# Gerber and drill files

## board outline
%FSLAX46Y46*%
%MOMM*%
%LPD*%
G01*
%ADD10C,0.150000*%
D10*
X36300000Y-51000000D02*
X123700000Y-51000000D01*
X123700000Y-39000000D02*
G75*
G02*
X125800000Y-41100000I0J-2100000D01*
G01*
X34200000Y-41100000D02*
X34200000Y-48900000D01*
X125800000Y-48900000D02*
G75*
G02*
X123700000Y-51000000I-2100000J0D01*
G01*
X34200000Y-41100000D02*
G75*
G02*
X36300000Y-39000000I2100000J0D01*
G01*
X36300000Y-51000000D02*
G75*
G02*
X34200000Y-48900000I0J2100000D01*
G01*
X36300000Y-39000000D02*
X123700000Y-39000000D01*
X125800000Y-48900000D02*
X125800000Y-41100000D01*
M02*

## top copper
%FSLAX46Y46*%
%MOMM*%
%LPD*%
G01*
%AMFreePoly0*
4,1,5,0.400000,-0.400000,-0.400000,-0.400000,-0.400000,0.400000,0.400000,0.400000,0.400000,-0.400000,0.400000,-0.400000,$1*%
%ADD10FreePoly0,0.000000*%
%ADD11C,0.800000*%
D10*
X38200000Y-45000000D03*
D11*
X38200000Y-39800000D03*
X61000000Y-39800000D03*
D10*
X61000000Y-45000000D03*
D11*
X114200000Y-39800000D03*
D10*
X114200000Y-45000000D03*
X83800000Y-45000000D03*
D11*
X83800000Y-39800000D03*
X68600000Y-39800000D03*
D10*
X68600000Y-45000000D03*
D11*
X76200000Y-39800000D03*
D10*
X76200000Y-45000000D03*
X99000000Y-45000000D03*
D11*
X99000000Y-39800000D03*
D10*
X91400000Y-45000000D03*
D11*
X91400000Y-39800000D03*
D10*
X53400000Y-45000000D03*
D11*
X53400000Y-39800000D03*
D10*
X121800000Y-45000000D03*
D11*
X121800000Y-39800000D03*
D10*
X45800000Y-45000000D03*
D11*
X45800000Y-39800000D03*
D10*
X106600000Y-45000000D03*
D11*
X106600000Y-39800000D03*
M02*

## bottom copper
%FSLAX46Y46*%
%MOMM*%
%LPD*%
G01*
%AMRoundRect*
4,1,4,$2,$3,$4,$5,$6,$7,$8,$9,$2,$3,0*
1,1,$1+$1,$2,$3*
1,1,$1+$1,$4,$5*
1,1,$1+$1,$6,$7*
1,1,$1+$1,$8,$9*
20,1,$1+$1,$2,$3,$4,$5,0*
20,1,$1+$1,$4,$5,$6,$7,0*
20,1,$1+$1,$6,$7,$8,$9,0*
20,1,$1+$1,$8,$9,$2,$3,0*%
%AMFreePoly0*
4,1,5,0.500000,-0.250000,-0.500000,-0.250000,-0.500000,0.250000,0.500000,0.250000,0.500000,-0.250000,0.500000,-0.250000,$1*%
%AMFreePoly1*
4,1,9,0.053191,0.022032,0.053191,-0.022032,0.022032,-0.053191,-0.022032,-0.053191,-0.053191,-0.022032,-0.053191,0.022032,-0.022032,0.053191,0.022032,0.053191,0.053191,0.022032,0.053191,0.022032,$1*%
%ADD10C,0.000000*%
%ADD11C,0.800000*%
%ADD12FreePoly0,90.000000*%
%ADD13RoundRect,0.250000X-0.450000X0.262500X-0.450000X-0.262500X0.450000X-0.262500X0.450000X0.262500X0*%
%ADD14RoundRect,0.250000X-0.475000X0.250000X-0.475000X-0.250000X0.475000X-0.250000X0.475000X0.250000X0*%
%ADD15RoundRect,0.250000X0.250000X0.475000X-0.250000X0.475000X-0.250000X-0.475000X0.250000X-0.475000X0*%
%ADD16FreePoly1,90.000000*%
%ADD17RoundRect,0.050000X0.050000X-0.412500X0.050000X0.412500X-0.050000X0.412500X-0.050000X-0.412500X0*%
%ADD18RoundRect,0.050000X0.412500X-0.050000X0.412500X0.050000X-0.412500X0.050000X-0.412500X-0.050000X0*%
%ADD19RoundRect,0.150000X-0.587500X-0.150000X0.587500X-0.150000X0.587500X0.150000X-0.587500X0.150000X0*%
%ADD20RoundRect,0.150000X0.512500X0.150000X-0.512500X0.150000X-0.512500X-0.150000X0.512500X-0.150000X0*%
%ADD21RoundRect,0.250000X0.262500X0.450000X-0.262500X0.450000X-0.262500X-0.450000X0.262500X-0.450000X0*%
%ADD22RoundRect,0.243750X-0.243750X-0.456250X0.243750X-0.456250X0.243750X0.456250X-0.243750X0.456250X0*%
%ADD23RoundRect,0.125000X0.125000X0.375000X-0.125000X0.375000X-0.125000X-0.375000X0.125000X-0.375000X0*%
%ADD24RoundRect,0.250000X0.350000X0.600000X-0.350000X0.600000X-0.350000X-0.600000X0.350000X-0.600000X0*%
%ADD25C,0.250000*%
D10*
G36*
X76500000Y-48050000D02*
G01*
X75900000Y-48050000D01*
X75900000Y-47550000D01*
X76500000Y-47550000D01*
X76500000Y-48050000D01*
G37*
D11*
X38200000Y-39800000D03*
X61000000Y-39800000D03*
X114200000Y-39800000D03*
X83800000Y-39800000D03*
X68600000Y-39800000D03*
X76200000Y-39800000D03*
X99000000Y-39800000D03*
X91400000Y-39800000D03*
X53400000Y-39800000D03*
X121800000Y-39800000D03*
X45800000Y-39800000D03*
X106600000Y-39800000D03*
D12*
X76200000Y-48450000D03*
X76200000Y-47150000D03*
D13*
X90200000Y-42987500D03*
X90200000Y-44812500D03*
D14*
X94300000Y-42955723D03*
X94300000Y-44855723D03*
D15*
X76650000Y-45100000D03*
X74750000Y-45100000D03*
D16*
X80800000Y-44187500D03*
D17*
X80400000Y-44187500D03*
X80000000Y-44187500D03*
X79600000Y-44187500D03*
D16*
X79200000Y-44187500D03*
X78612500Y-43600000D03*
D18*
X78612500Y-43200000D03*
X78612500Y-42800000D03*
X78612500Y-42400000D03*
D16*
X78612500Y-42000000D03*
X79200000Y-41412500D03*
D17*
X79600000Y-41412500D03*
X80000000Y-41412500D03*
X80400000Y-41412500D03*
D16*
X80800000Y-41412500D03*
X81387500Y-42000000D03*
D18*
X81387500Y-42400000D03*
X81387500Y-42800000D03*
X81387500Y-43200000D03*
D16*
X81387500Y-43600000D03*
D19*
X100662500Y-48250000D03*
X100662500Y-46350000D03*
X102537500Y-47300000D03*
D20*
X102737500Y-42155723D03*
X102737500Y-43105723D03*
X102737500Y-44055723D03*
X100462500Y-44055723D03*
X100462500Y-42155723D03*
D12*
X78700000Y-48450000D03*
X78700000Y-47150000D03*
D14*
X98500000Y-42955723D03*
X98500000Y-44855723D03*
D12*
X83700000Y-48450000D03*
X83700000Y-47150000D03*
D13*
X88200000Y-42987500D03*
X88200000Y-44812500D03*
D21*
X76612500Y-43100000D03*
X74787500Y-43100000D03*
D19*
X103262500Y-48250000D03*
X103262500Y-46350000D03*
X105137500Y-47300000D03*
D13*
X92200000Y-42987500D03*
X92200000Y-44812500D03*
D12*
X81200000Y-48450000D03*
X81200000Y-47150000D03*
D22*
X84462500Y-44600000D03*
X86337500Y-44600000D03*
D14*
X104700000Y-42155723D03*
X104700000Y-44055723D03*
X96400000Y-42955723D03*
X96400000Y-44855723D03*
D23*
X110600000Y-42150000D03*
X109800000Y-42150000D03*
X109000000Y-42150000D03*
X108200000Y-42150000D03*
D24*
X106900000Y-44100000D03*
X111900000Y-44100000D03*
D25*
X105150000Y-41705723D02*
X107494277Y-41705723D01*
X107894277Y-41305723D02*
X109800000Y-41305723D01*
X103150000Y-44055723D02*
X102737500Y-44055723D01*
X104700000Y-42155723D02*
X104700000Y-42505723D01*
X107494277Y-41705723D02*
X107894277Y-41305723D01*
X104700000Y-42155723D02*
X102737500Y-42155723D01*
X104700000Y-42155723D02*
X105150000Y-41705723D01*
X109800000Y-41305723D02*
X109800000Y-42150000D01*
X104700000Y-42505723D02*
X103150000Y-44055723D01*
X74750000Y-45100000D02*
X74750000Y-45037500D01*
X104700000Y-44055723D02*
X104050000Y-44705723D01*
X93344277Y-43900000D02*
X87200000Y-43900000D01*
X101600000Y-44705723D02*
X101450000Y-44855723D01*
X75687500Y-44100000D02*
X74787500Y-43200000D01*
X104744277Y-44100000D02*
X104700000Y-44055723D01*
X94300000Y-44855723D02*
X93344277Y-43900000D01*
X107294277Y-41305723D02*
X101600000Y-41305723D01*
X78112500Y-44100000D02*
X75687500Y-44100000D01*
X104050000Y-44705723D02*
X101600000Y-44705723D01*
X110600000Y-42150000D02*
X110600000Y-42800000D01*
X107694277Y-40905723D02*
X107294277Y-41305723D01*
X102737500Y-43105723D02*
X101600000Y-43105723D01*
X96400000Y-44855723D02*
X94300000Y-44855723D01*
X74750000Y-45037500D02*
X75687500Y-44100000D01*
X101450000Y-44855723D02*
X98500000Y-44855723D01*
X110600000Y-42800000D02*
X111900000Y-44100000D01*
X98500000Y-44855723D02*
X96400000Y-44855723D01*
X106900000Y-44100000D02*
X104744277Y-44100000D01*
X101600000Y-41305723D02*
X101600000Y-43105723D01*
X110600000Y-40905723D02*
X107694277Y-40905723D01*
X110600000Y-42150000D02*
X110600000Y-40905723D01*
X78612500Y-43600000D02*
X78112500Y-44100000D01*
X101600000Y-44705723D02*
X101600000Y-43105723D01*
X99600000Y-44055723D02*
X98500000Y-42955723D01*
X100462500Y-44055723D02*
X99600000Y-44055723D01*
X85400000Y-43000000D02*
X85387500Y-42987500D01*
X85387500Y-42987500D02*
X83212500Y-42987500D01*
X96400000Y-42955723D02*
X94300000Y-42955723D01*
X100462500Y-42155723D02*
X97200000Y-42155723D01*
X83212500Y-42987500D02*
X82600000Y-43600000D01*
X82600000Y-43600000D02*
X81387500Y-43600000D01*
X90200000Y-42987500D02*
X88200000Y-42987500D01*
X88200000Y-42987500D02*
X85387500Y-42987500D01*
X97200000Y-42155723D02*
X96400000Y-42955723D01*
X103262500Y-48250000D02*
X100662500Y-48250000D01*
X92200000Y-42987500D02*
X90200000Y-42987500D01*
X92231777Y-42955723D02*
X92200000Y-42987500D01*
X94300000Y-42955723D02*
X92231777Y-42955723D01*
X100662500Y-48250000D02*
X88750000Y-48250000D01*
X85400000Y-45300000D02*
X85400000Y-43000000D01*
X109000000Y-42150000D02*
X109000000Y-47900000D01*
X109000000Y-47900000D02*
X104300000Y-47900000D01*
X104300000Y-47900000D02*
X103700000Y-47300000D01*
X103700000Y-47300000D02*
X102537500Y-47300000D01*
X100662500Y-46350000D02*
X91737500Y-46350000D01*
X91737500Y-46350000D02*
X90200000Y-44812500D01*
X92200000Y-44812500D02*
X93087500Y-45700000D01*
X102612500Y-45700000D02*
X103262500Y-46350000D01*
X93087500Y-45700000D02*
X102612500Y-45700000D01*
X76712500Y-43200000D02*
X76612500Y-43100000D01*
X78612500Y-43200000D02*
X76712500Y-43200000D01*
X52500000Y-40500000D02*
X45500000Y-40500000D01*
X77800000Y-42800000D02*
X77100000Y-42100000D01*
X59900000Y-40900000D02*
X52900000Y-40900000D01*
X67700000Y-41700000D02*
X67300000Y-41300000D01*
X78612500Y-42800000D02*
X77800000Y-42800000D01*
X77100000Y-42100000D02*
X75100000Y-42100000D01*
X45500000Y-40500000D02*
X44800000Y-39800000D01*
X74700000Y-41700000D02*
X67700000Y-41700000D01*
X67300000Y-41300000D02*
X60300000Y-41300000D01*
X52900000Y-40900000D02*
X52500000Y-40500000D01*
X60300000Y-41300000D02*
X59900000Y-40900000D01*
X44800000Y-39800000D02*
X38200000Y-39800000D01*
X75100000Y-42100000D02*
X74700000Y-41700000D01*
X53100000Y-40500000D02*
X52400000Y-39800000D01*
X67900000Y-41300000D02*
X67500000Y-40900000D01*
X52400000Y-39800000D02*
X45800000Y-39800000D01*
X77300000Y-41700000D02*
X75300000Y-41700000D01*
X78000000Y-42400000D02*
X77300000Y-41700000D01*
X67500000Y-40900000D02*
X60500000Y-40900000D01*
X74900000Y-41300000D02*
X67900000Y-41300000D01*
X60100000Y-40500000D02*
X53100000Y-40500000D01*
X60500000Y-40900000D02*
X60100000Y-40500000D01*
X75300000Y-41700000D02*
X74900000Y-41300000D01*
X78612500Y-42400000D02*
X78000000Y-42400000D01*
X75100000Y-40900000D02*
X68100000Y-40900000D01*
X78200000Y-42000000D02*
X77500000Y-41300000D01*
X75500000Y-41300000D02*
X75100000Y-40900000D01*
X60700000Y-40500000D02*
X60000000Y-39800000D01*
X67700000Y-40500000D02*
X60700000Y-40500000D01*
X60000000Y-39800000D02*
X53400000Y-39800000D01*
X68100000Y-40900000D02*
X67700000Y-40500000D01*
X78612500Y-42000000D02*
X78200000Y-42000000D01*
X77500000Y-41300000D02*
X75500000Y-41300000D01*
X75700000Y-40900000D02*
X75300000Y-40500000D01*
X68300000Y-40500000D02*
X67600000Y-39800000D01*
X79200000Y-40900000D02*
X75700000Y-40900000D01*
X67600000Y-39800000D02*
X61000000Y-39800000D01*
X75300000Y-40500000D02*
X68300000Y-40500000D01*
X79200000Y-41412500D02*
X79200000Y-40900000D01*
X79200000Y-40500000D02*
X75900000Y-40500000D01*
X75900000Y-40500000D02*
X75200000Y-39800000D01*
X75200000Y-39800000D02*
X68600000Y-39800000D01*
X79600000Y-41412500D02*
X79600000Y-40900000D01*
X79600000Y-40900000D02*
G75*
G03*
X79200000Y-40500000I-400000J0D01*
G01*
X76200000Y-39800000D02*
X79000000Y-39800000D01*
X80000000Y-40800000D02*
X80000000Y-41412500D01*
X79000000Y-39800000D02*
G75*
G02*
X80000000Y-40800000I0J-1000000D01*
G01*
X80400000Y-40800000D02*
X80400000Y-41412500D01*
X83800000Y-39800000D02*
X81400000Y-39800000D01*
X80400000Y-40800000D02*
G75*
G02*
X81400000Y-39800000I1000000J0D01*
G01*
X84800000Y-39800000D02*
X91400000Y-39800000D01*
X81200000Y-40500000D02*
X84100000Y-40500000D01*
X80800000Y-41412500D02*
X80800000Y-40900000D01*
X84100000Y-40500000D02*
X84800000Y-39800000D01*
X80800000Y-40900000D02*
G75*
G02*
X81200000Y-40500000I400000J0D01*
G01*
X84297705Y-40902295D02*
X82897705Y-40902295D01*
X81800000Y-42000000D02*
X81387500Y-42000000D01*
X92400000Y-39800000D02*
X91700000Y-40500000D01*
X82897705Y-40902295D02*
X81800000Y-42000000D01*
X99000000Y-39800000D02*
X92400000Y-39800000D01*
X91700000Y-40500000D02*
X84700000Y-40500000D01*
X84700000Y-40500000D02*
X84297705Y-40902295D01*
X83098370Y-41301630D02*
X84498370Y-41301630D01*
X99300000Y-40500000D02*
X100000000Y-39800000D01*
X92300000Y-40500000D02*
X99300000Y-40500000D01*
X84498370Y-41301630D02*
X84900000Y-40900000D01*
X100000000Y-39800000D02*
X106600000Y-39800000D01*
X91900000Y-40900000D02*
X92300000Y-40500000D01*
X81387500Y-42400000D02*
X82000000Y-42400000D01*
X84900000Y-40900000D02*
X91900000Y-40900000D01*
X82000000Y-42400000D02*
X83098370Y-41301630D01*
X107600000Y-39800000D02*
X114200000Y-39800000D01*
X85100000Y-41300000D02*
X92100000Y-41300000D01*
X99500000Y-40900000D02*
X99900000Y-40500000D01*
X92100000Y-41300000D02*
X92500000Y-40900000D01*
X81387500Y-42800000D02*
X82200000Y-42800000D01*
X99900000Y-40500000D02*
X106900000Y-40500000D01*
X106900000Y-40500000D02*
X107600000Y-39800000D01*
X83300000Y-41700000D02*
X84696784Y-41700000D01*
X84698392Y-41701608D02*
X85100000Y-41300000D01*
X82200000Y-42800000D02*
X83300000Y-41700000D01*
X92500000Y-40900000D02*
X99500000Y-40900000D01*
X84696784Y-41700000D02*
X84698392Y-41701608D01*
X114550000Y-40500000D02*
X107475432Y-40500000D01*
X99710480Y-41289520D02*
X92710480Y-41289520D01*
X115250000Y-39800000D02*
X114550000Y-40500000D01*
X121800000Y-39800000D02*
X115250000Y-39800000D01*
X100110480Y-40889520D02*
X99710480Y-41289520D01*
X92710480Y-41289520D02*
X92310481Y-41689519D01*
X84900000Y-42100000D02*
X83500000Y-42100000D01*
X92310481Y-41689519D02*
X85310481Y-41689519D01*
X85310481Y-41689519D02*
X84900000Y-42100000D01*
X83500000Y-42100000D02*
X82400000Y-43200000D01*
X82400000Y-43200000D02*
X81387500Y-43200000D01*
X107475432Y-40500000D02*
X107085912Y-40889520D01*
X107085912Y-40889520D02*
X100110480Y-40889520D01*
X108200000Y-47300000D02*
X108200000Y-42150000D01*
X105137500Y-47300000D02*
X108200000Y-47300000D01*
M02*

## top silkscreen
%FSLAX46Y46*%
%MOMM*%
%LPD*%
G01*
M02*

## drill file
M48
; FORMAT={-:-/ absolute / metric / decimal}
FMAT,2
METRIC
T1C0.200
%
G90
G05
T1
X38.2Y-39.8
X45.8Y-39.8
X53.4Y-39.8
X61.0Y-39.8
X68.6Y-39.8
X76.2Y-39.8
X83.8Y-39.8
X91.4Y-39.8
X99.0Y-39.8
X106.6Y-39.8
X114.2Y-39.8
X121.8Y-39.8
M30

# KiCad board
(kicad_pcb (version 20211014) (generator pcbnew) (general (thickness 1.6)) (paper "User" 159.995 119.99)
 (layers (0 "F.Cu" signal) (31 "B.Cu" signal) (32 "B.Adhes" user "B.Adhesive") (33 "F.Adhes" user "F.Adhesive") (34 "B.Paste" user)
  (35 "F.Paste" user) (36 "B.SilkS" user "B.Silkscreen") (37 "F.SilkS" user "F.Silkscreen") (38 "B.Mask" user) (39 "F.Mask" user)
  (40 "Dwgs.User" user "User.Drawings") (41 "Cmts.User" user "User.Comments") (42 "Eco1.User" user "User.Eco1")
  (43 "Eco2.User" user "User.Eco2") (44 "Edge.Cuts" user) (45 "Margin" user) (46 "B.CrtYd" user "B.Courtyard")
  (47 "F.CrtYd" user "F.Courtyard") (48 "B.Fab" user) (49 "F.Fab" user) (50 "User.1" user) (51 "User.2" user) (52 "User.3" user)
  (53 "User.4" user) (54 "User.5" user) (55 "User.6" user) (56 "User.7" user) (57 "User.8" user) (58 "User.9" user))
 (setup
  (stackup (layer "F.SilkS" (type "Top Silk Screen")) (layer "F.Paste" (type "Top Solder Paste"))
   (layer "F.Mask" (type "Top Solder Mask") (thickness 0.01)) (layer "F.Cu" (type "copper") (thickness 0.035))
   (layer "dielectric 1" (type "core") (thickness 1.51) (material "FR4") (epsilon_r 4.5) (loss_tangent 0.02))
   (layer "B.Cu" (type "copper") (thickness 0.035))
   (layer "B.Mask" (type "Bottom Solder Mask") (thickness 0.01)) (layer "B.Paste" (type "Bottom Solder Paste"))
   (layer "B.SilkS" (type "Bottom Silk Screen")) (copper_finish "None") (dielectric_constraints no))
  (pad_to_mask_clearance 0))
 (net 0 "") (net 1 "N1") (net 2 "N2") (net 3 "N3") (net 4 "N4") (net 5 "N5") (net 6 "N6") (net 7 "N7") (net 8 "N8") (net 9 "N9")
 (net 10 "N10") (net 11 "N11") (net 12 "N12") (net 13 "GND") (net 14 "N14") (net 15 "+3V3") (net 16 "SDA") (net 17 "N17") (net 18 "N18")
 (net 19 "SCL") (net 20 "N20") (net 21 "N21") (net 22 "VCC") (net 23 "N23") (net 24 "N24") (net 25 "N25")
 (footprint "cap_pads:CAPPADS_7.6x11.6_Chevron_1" (layer "F.Cu") (at 38.2 45)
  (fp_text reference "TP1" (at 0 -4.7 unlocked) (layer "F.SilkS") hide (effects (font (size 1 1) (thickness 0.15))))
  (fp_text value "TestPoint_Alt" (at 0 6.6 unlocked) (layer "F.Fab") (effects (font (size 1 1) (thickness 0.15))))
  (pad "1" smd custom (at 0 0) (size 0.8 0.8) (layers "F.Cu") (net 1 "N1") (options (clearance outline) (anchor rect)) (primitives))
  (pad "1" thru_hole circle (at 0 -5.2) (size 0.8 0.8) (drill 0.2) (layers *.Cu) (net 1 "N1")))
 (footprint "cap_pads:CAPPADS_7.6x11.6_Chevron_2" (layer "F.Cu") (at 61 45)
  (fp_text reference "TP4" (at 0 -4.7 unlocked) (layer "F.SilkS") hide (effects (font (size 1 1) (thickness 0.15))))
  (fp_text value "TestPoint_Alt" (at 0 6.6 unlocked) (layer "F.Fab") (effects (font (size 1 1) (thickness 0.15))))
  (pad "1" thru_hole circle (at 0 -5.2) (size 0.8 0.8) (drill 0.2) (layers *.Cu) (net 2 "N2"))
  (pad "1" smd custom (at 0 0) (size 0.8 0.8) (layers "F.Cu") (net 2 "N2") (options (clearance outline) (anchor rect)) (primitives)))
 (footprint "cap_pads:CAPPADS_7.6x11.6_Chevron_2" (layer "F.Cu") (at 114.2 45)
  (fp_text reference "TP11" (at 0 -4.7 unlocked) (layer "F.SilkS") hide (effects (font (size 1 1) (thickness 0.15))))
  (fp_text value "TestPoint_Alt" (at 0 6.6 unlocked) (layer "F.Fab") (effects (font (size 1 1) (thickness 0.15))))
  (pad "1" thru_hole circle (at 0 -5.2) (size 0.8 0.8) (drill 0.2) (layers *.Cu) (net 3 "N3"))
  (pad "1" smd custom (at 0 0) (size 0.8 0.8) (layers "F.Cu") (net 3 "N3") (options (clearance outline) (anchor rect)) (primitives)))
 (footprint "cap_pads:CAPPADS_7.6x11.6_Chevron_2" (layer "F.Cu") (at 83.8 45)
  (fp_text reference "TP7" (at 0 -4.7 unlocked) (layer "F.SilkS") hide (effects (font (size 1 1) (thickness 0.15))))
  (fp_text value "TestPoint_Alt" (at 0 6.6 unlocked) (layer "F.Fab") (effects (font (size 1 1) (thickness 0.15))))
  (pad "1" smd custom (at 0 0) (size 0.8 0.8) (layers "F.Cu") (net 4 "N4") (options (clearance outline) (anchor rect)) (primitives))
  (pad "1" thru_hole circle (at 0 -5.2) (size 0.8 0.8) (drill 0.2) (layers *.Cu) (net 4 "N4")))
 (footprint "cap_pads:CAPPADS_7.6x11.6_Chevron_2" (layer "F.Cu") (at 68.6 45)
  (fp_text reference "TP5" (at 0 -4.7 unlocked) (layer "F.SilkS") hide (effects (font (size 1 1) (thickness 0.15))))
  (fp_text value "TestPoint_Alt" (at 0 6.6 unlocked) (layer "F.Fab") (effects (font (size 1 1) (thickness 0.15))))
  (pad "1" thru_hole circle (at 0 -5.2) (size 0.8 0.8) (drill 0.2) (layers *.Cu) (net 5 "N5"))
  (pad "1" smd custom (at 0 0) (size 0.8 0.8) (layers "F.Cu") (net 5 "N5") (options (clearance outline) (anchor rect)) (primitives)))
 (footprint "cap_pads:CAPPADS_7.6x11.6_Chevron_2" (layer "F.Cu") (at 76.2 45)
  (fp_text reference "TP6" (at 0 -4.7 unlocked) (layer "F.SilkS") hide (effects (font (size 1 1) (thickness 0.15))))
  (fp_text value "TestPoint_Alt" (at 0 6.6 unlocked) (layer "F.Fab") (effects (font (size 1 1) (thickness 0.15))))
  (pad "1" thru_hole circle (at 0 -5.2) (size 0.8 0.8) (drill 0.2) (layers *.Cu) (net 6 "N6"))
  (pad "1" smd custom (at 0 0) (size 0.8 0.8) (layers "F.Cu") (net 6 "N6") (options (clearance outline) (anchor rect)) (primitives)))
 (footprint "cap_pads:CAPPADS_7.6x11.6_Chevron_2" (layer "F.Cu") (at 99 45)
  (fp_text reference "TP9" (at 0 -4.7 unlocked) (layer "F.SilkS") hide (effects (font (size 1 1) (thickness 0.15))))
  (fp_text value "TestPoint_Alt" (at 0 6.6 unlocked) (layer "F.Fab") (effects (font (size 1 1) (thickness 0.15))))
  (pad "1" smd custom (at 0 0) (size 0.8 0.8) (layers "F.Cu") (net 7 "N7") (options (clearance outline) (anchor rect)) (primitives))
  (pad "1" thru_hole circle (at 0 -5.2) (size 0.8 0.8) (drill 0.2) (layers *.Cu) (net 7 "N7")))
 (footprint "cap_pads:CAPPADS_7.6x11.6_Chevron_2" (layer "F.Cu") (at 91.4 45)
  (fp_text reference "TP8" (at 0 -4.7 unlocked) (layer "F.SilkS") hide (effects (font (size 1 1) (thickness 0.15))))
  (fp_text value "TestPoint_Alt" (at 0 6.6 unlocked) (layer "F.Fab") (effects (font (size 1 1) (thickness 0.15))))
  (pad "1" smd custom (at 0 0) (size 0.8 0.8) (layers "F.Cu") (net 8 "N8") (options (clearance outline) (anchor rect)) (primitives))
  (pad "1" thru_hole circle (at 0 -5.2) (size 0.8 0.8) (drill 0.2) (layers *.Cu) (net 8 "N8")))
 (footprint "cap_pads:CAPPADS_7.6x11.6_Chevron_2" (layer "F.Cu") (at 53.4 45)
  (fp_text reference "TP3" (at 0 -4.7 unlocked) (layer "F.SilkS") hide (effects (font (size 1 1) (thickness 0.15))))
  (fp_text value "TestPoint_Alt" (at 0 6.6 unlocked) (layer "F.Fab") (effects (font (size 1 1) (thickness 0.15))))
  (pad "1" smd custom (at 0 0) (size 0.8 0.8) (layers "F.Cu") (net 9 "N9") (options (clearance outline) (anchor rect)) (primitives))
  (pad "1" thru_hole circle (at 0 -5.2) (size 0.8 0.8) (drill 0.2) (layers *.Cu) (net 9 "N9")))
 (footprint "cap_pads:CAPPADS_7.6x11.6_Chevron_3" (layer "F.Cu") (at 121.8 45)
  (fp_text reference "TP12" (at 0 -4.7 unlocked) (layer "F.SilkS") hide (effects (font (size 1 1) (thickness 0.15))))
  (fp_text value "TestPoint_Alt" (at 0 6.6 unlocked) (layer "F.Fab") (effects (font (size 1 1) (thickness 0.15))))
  (pad "1" smd custom (at 0 0) (size 0.8 0.8) (layers "F.Cu") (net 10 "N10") (options (clearance outline) (anchor rect)) (primitives))
  (pad "1" thru_hole circle (at 0 -5.2) (size 0.8 0.8) (drill 0.2) (layers *.Cu) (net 10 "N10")))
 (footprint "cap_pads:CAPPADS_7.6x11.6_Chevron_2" (layer "F.Cu") (at 45.8 45)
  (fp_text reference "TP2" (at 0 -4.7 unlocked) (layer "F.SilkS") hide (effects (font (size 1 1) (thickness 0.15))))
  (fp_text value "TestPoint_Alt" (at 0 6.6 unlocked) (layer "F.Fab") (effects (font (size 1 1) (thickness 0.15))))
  (pad "1" smd custom (at 0 0) (size 0.8 0.8) (layers "F.Cu") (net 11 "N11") (options (clearance outline) (anchor rect)) (primitives))
  (pad "1" thru_hole circle (at 0 -5.2) (size 0.8 0.8) (drill 0.2) (layers *.Cu) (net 11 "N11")))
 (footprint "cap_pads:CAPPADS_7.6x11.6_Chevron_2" (layer "F.Cu") (at 106.6 45)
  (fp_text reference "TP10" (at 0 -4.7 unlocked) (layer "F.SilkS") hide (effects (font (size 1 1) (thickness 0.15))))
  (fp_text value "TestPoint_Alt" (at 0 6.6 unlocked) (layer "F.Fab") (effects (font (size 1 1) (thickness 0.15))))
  (pad "1" smd custom (at 0 0) (size 0.8 0.8) (layers "F.Cu") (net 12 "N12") (options (clearance outline) (anchor rect)) (primitives))
  (pad "1" thru_hole circle (at 0 -5.2) (size 0.8 0.8) (drill 0.2) (layers *.Cu) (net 12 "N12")))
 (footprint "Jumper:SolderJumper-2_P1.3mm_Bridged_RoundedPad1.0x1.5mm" (layer "B.Cu") (at 76.2 47.8 90)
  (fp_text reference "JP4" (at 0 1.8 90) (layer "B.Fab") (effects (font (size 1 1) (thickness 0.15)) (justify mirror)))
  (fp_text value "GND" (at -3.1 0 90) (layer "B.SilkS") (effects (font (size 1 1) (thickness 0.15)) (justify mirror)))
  (fp_poly (pts (xy 0.25 0.3) (xy -0.25 0.3) (xy -0.25 -0.3) (xy 0.25 -0.3)) (layer "B.Cu") (width 0) (fill solid))
  (pad "1" smd custom (at -0.65 0 90) (size 1 0.5) (layers "B.Cu" "B.Mask") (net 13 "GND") (zone_connect 2)
   (options (clearance outline) (anchor rect)) (primitives))
  (pad "2" smd custom (at 0.65 0 90) (size 1 0.5) (layers "B.Cu" "B.Mask") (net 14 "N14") (zone_connect 2)
   (options (clearance outline) (anchor rect)) (primitives)))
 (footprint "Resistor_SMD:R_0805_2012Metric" (layer "B.Cu") (at 90.2 43.9 -90)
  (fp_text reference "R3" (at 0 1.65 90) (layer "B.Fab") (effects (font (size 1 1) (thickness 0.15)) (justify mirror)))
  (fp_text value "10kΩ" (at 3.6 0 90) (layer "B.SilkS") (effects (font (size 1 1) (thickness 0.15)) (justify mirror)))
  (pad "1" smd roundrect (at -0.9125 0 270) (size 1.025 1.4) (layers "B.Cu" "B.Paste" "B.Mask") (roundrect_rratio 0.243902) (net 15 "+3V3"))
  (pad "2" smd roundrect (at 0.9125 0 270) (size 1.025 1.4) (layers "B.Cu" "B.Paste" "B.Mask") (roundrect_rratio 0.243902) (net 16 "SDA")))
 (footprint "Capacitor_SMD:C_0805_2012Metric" (layer "B.Cu") (at 94.3 43.905723 -90)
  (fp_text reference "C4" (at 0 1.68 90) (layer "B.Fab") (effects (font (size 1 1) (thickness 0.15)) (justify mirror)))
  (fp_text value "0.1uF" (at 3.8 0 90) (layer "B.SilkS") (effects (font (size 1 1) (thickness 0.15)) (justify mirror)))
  (pad "1" smd roundrect (at -0.95 0 270) (size 1 1.45) (layers "B.Cu" "B.Paste" "B.Mask") (roundrect_rratio 0.25) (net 15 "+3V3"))
  (pad "2" smd roundrect (at 0.95 0 270) (size 1 1.45) (layers "B.Cu" "B.Paste" "B.Mask") (roundrect_rratio 0.25) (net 13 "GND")))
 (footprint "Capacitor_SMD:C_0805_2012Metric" (layer "B.Cu") (at 75.7 45.1 180)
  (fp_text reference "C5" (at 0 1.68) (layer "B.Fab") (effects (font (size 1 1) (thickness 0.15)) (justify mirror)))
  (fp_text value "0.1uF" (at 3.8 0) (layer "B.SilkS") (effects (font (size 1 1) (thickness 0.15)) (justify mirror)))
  (pad "1" smd roundrect (at -0.95 0 180) (size 1 1.45) (layers "B.Cu" "B.Paste" "B.Mask") (roundrect_rratio 0.25) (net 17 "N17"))
  (pad "2" smd roundrect (at 0.95 0 180) (size 1 1.45) (layers "B.Cu" "B.Paste" "B.Mask") (roundrect_rratio 0.25) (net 13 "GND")))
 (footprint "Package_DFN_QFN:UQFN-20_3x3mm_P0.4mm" (layer "B.Cu") (at 80 42.8 90)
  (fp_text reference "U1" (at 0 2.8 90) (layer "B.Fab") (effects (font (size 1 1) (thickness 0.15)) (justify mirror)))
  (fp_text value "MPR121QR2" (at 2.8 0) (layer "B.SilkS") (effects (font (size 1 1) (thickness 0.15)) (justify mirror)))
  (pad "1" smd custom (at -1.3875 0.8 90) (size 0.115147 0.115147) (layers "B.Cu" "B.Paste" "B.Mask") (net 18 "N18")
   (options (clearance outline) (anchor circle)) (primitives))
  (pad "2" smd roundrect (at -1.3875 0.4 90) (size 0.925 0.2) (layers "B.Cu" "B.Paste" "B.Mask") (roundrect_rratio 0.25) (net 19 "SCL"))
  (pad "3" smd roundrect (at -1.3875 0 90) (size 0.925 0.2) (layers "B.Cu" "B.Paste" "B.Mask") (roundrect_rratio 0.25) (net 16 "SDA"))
  (pad "4" smd roundrect (at -1.3875 -0.4 90) (size 0.925 0.2) (layers "B.Cu" "B.Paste" "B.Mask") (roundrect_rratio 0.25) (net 14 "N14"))
  (pad "5" smd custom (at -1.3875 -0.8 90) (size 0.115147 0.115147) (layers "B.Cu" "B.Paste" "B.Mask") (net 17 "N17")
   (options (clearance outline) (anchor circle)) (primitives))
  (pad "6" smd custom (at -0.8 -1.3875 90) (size 0.115147 0.115147) (layers "B.Cu" "B.Paste" "B.Mask") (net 13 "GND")
   (options (clearance outline) (anchor circle)) (primitives))
  (pad "7" smd roundrect (at -0.4 -1.3875 90) (size 0.2 0.925) (layers "B.Cu" "B.Paste" "B.Mask") (roundrect_rratio 0.25) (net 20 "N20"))
  (pad "8" smd roundrect (at 0 -1.3875 90) (size 0.2 0.925) (layers "B.Cu" "B.Paste" "B.Mask") (roundrect_rratio 0.25) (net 1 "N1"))
  (pad "9" smd roundrect (at 0.4 -1.3875 90) (size 0.2 0.925) (layers "B.Cu" "B.Paste" "B.Mask") (roundrect_rratio 0.25) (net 11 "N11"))
  (pad "10" smd custom (at 0.8 -1.3875 90) (size 0.115147 0.115147) (layers "B.Cu" "B.Paste" "B.Mask") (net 9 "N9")
   (options (clearance outline) (anchor circle)) (primitives))
  (pad "11" smd custom (at 1.3875 -0.8 90) (size 0.115147 0.115147) (layers "B.Cu" "B.Paste" "B.Mask") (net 2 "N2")
   (options (clearance outline) (anchor circle)) (primitives))
  (pad "12" smd roundrect (at 1.3875 -0.4 90) (size 0.925 0.2) (layers "B.Cu" "B.Paste" "B.Mask") (roundrect_rratio 0.25) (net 5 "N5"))
  (pad "13" smd roundrect (at 1.3875 0 90) (size 0.925 0.2) (layers "B.Cu" "B.Paste" "B.Mask") (roundrect_rratio 0.25) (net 6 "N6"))
  (pad "14" smd roundrect (at 1.3875 0.4 90) (size 0.925 0.2) (layers "B.Cu" "B.Paste" "B.Mask") (roundrect_rratio 0.25) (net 4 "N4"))
  (pad "15" smd custom (at 1.3875 0.8 90) (size 0.115147 0.115147) (layers "B.Cu" "B.Paste" "B.Mask") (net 8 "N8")
   (options (clearance outline) (anchor circle)) (primitives))
  (pad "16" smd custom (at 0.8 1.3875 90) (size 0.115147 0.115147) (layers "B.Cu" "B.Paste" "B.Mask") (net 7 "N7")
   (options (clearance outline) (anchor circle)) (primitives))
  (pad "17" smd roundrect (at 0.4 1.3875 90) (size 0.2 0.925) (layers "B.Cu" "B.Paste" "B.Mask") (roundrect_rratio 0.25) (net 12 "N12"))
  (pad "18" smd roundrect (at 0 1.3875 90) (size 0.2 0.925) (layers "B.Cu" "B.Paste" "B.Mask") (roundrect_rratio 0.25) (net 3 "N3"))
  (pad "19" smd roundrect (at -0.4 1.3875 90) (size 0.2 0.925) (layers "B.Cu" "B.Paste" "B.Mask") (roundrect_rratio 0.25) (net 10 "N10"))
  (pad "20" smd custom (at -0.8 1.3875 90) (size 0.115147 0.115147) (layers "B.Cu" "B.Paste" "B.Mask") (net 15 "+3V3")
   (options (clearance outline) (anchor circle)) (primitives)))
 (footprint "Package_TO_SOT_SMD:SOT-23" (layer "B.Cu") (at 101.6 47.3)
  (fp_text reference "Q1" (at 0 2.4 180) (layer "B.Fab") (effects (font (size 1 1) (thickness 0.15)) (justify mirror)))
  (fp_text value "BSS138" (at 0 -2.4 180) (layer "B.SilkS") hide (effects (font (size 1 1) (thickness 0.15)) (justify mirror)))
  (pad "1" smd roundrect (at -0.9375 0.95) (size 1.475 0.6) (layers "B.Cu" "B.Paste" "B.Mask") (roundrect_rratio 0.25) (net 15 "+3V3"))
  (pad "2" smd roundrect (at -0.9375 -0.95) (size 1.475 0.6) (layers "B.Cu" "B.Paste" "B.Mask") (roundrect_rratio 0.25) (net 16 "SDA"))
  (pad "3" smd roundrect (at 0.9375 0) (size 1.475 0.6) (layers "B.Cu" "B.Paste" "B.Mask") (roundrect_rratio 0.25) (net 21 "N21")))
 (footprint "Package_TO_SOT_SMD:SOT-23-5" (layer "B.Cu") (at 101.6 43.105723 180)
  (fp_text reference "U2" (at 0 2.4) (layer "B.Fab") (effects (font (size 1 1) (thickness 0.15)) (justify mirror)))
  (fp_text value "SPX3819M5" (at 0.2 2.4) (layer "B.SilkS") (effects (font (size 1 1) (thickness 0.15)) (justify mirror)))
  (pad "1" smd roundrect (at -1.1375 0.95 180) (size 1.325 0.6) (layers "B.Cu" "B.Paste" "B.Mask") (roundrect_rratio 0.25) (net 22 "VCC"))
  (pad "2" smd roundrect (at -1.1375 0 180) (size 1.325 0.6) (layers "B.Cu" "B.Paste" "B.Mask") (roundrect_rratio 0.25) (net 13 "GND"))
  (pad "3" smd roundrect (at -1.1375 -0.95 180) (size 1.325 0.6) (layers "B.Cu" "B.Paste" "B.Mask") (roundrect_rratio 0.25) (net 22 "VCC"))
  (pad "4" smd roundrect (at 1.1375 -0.95 180) (size 1.325 0.6) (layers "B.Cu" "B.Paste" "B.Mask") (roundrect_rratio 0.25) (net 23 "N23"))
  (pad "5" smd roundrect (at 1.1375 0.95 180) (size 1.325 0.6) (layers "B.Cu" "B.Paste" "B.Mask") (roundrect_rratio 0.25) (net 15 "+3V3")))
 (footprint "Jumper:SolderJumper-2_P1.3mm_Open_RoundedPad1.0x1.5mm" (layer "B.Cu") (at 78.7 47.8 90)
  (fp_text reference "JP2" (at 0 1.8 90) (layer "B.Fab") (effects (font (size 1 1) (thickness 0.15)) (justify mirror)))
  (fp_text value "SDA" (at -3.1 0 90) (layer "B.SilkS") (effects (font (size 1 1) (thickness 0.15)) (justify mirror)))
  (pad "1" smd custom (at -0.65 0 90) (size 1 0.5) (layers "B.Cu" "B.Mask") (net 16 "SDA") (zone_connect 2)
   (options (clearance outline) (anchor rect)) (primitives))
  (pad "2" smd custom (at 0.65 0 90) (size 1 0.5) (layers "B.Cu" "B.Mask") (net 14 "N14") (zone_connect 2)
   (options (clearance outline) (anchor rect)) (primitives)))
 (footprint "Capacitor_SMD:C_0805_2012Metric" (layer "B.Cu") (at 98.5 43.905723 -90)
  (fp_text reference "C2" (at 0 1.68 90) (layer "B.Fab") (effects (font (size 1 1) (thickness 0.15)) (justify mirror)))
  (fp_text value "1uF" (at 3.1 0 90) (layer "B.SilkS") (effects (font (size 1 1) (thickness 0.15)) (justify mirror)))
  (pad "1" smd roundrect (at -0.95 0 270) (size 1 1.45) (layers "B.Cu" "B.Paste" "B.Mask") (roundrect_rratio 0.25) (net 23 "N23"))
  (pad "2" smd roundrect (at 0.95 0 270) (size 1 1.45) (layers "B.Cu" "B.Paste" "B.Mask") (roundrect_rratio 0.25) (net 13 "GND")))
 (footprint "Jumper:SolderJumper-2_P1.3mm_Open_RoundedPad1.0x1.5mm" (layer "B.Cu") (at 83.7 47.8 90)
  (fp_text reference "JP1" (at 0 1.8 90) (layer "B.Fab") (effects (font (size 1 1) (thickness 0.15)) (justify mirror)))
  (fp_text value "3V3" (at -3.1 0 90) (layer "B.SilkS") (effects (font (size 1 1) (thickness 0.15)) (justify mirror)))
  (pad "1" smd custom (at -0.65 0 90) (size 1 0.5) (layers "B.Cu" "B.Mask") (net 15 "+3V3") (zone_connect 2)
   (options (clearance outline) (anchor rect)) (primitives))
  (pad "2" smd custom (at 0.65 0 90) (size 1 0.5) (layers "B.Cu" "B.Mask") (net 14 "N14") (zone_connect 2)
   (options (clearance outline) (anchor rect)) (primitives)))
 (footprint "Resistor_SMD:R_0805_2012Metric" (layer "B.Cu") (at 88.2 43.9 -90)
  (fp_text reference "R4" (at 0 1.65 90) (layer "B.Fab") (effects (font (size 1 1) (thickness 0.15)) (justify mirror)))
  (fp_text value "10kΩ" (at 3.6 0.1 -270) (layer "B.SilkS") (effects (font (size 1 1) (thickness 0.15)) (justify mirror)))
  (pad "1" smd roundrect (at -0.9125 0 270) (size 1.025 1.4) (layers "B.Cu" "B.Paste" "B.Mask") (roundrect_rratio 0.243902) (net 15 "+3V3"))
  (pad "2" smd roundrect (at 0.9125 0 270) (size 1.025 1.4) (layers "B.Cu" "B.Paste" "B.Mask") (roundrect_rratio 0.243902) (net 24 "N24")))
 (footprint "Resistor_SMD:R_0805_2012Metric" (layer "B.Cu") (at 75.7 43.1 180)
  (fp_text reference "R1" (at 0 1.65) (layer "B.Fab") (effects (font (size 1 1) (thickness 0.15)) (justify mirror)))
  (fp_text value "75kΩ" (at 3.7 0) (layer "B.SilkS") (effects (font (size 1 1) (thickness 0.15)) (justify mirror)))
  (pad "1" smd roundrect (at -0.9125 0 180) (size 1.025 1.4) (layers "B.Cu" "B.Paste" "B.Mask") (roundrect_rratio 0.243902) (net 20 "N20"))
  (pad "2" smd roundrect (at 0.9125 0 180) (size 1.025 1.4) (layers "B.Cu" "B.Paste" "B.Mask") (roundrect_rratio 0.243902) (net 13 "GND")))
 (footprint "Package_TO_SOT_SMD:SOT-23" (layer "B.Cu") (at 104.2 47.3)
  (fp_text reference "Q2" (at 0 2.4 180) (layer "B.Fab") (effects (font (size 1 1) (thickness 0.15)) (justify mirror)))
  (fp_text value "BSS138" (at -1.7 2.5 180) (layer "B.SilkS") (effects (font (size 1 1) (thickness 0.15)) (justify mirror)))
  (pad "1" smd roundrect (at -0.9375 0.95) (size 1.475 0.6) (layers "B.Cu" "B.Paste" "B.Mask") (roundrect_rratio 0.25) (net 15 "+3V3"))
  (pad "2" smd roundrect (at -0.9375 -0.95) (size 1.475 0.6) (layers "B.Cu" "B.Paste" "B.Mask") (roundrect_rratio 0.25) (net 19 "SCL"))
  (pad "3" smd roundrect (at 0.9375 0) (size 1.475 0.6) (layers "B.Cu" "B.Paste" "B.Mask") (roundrect_rratio 0.25) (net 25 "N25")))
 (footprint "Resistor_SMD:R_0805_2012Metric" (layer "B.Cu") (at 92.2 43.9 -90)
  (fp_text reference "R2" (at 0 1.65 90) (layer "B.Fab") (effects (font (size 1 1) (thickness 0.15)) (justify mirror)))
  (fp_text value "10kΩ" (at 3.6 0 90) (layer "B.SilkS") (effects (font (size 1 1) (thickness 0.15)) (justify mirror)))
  (pad "1" smd roundrect (at -0.9125 0 270) (size 1.025 1.4) (layers "B.Cu" "B.Paste" "B.Mask") (roundrect_rratio 0.243902) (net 15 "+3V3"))
  (pad "2" smd roundrect (at 0.9125 0 270) (size 1.025 1.4) (layers "B.Cu" "B.Paste" "B.Mask") (roundrect_rratio 0.243902) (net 19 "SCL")))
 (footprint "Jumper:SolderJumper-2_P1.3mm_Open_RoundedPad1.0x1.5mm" (layer "B.Cu") (at 81.2 47.8 90)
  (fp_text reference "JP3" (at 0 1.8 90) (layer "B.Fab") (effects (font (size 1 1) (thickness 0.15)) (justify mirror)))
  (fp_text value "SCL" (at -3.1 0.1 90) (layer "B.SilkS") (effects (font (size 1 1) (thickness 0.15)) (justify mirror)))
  (pad "1" smd custom (at -0.65 0 90) (size 1 0.5) (layers "B.Cu" "B.Mask") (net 19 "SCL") (zone_connect 2)
   (options (clearance outline) (anchor rect)) (primitives))
  (pad "2" smd custom (at 0.65 0 90) (size 1 0.5) (layers "B.Cu" "B.Mask") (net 14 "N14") (zone_connect 2)
   (options (clearance outline) (anchor rect)) (primitives)))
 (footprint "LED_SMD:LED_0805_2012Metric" (layer "B.Cu") (at 85.4 44.6)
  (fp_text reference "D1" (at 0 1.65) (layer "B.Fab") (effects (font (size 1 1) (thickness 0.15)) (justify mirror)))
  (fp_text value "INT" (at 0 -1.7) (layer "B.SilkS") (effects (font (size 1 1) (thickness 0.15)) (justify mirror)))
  (pad "1" smd roundrect (at -0.9375 0) (size 0.975 1.4) (layers "B.Cu" "B.Paste" "B.Mask") (roundrect_rratio 0.25) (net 18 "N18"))
  (pad "2" smd roundrect (at 0.9375 0) (size 0.975 1.4) (layers "B.Cu" "B.Paste" "B.Mask") (roundrect_rratio 0.25) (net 24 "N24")))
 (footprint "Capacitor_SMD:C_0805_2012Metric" (layer "B.Cu") (at 104.7 43.105723 -90)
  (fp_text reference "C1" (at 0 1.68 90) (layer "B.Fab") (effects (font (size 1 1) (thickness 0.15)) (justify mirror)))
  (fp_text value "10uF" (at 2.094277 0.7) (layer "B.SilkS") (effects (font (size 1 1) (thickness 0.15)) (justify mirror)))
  (pad "1" smd roundrect (at -0.95 0 270) (size 1 1.45) (layers "B.Cu" "B.Paste" "B.Mask") (roundrect_rratio 0.25) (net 22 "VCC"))
  (pad "2" smd roundrect (at 0.95 0 270) (size 1 1.45) (layers "B.Cu" "B.Paste" "B.Mask") (roundrect_rratio 0.25) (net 13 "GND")))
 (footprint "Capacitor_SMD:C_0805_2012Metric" (layer "B.Cu") (at 96.4 43.905723 -90)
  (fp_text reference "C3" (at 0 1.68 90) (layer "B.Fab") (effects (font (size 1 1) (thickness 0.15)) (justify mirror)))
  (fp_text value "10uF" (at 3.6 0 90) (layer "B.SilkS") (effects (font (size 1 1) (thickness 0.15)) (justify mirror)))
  (pad "1" smd roundrect (at -0.95 0 270) (size 1 1.45) (layers "B.Cu" "B.Paste" "B.Mask") (roundrect_rratio 0.25) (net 15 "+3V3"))
  (pad "2" smd roundrect (at 0.95 0 270) (size 1 1.45) (layers "B.Cu" "B.Paste" "B.Mask") (roundrect_rratio 0.25) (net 13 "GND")))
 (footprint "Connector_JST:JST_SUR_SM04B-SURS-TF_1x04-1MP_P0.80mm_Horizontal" (layer "B.Cu") (at 109.4 43.3 180)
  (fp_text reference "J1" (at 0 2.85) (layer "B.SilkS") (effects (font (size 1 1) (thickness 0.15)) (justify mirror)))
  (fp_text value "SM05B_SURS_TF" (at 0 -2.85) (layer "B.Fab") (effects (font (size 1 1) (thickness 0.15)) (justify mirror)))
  (pad "1" smd roundrect (at -1.2 1.15 180) (size 0.5 1) (layers "B.Cu" "B.Paste" "B.Mask") (roundrect_rratio 0.25) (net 13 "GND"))
  (pad "2" smd roundrect (at -0.4 1.15 180) (size 0.5 1) (layers "B.Cu" "B.Paste" "B.Mask") (roundrect_rratio 0.25) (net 22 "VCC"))
  (pad "3" smd roundrect (at 0.4 1.15 180) (size 0.5 1) (layers "B.Cu" "B.Paste" "B.Mask") (roundrect_rratio 0.25) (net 21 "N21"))
  (pad "4" smd roundrect (at 1.2 1.15 180) (size 0.5 1) (layers "B.Cu" "B.Paste" "B.Mask") (roundrect_rratio 0.25) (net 25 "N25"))
  (pad "MP" smd roundrect (at 2.5 -0.8 180) (size 1.2 1.7) (layers "B.Cu" "B.Paste" "B.Mask") (roundrect_rratio 0.208333) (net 13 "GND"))
  (pad "MP" smd roundrect (at -2.5 -0.8 180) (size 1.2 1.7) (layers "B.Cu" "B.Paste" "B.Mask") (roundrect_rratio 0.208333) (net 13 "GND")))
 (gr_line (start 36.3 51) (end 123.7 51) (layer "Edge.Cuts") (width 0.15))
 (gr_arc (start 123.7 39) (mid 125.184924 39.615076) (end 125.8 41.1) (layer "Edge.Cuts") (width 0.15))
 (gr_line (start 34.2 41.1) (end 34.2 48.9) (layer "Edge.Cuts") (width 0.15))
 (gr_arc (start 125.8 48.9) (mid 125.184924 50.384924) (end 123.7 51) (layer "Edge.Cuts") (width 0.15))
 (gr_arc (start 34.2 41.1) (mid 34.815076 39.615076) (end 36.3 39) (layer "Edge.Cuts") (width 0.15))
 (gr_arc (start 36.3 51) (mid 34.815076 50.384924) (end 34.2 48.9) (layer "Edge.Cuts") (width 0.15))
 (gr_line (start 36.3 39) (end 123.7 39) (layer "Edge.Cuts") (width 0.15))
 (gr_line (start 125.8 48.9) (end 125.8 41.1) (layer "Edge.Cuts") (width 0.15))
 (segment (start 105.15 41.705723) (end 107.494277 41.705723) (width 0.25) (layer "B.Cu") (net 22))
 (segment (start 107.894277 41.305723) (end 109.8 41.305723) (width 0.25) (layer "B.Cu") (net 22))
 (segment (start 103.15 44.055723) (end 102.7375 44.055723) (width 0.25) (layer "B.Cu") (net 22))
 (segment (start 104.7 42.155723) (end 104.7 42.505723) (width 0.25) (layer "B.Cu") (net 22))
 (segment (start 107.494277 41.705723) (end 107.894277 41.305723) (width 0.25) (layer "B.Cu") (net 22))
 (segment (start 104.7 42.155723) (end 102.7375 42.155723) (width 0.25) (layer "B.Cu") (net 22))
 (segment (start 104.7 42.155723) (end 105.15 41.705723) (width 0.25) (layer "B.Cu") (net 22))
 (segment (start 109.8 41.305723) (end 109.8 42.15) (width 0.25) (layer "B.Cu") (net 22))
 (segment (start 104.7 42.505723) (end 103.15 44.055723) (width 0.25) (layer "B.Cu") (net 22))
 (segment (start 74.75 45.1) (end 74.75 45.0375) (width 0.25) (layer "B.Cu") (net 13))
 (segment (start 104.7 44.055723) (end 104.05 44.705723) (width 0.25) (layer "B.Cu") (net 13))
 (segment (start 93.344277 43.9) (end 87.2 43.9) (width 0.25) (layer "B.Cu") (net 13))
 (segment (start 101.6 44.705723) (end 101.45 44.855723) (width 0.25) (layer "B.Cu") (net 13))
 (segment (start 75.6875 44.1) (end 74.7875 43.2) (width 0.25) (layer "B.Cu") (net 13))
 (segment (start 104.744277 44.1) (end 104.7 44.055723) (width 0.25) (layer "B.Cu") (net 13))
 (segment (start 94.3 44.855723) (end 93.344277 43.9) (width 0.25) (layer "B.Cu") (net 13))
 (segment (start 107.294277 41.305723) (end 101.6 41.305723) (width 0.25) (layer "B.Cu") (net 13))
 (segment (start 78.1125 44.1) (end 75.6875 44.1) (width 0.25) (layer "B.Cu") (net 13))
 (segment (start 104.05 44.705723) (end 101.6 44.705723) (width 0.25) (layer "B.Cu") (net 13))
 (segment (start 110.6 42.15) (end 110.6 42.8) (width 0.25) (layer "B.Cu") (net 13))
 (segment (start 107.694277 40.905723) (end 107.294277 41.305723) (width 0.25) (layer "B.Cu") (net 13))
 (segment (start 102.7375 43.105723) (end 101.6 43.105723) (width 0.25) (layer "B.Cu") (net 13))
 (segment (start 96.4 44.855723) (end 94.3 44.855723) (width 0.25) (layer "B.Cu") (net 13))
 (segment (start 74.75 45.0375) (end 75.6875 44.1) (width 0.25) (layer "B.Cu") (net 13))
 (segment (start 101.45 44.855723) (end 98.5 44.855723) (width 0.25) (layer "B.Cu") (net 13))
 (segment (start 110.6 42.8) (end 111.9 44.1) (width 0.25) (layer "B.Cu") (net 13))
 (segment (start 98.5 44.855723) (end 96.4 44.855723) (width 0.25) (layer "B.Cu") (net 13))
 (segment (start 106.9 44.1) (end 104.744277 44.1) (width 0.25) (layer "B.Cu") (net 13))
 (segment (start 101.6 41.305723) (end 101.6 43.105723) (width 0.25) (layer "B.Cu") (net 13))
 (segment (start 110.6 40.905723) (end 107.694277 40.905723) (width 0.25) (layer "B.Cu") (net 13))
 (segment (start 110.6 42.15) (end 110.6 40.905723) (width 0.25) (layer "B.Cu") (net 13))
 (segment (start 78.6125 43.6) (end 78.1125 44.1) (width 0.25) (layer "B.Cu") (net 13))
 (segment (start 101.6 44.705723) (end 101.6 43.105723) (width 0.25) (layer "B.Cu") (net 13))
 (segment (start 99.6 44.055723) (end 98.5 42.955723) (width 0.25) (layer "B.Cu") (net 23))
 (segment (start 100.4625 44.055723) (end 99.6 44.055723) (width 0.25) (layer "B.Cu") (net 23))
 (segment (start 85.4 43) (end 85.3875 42.9875) (width 0.25) (layer "B.Cu") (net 15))
 (segment (start 85.3875 42.9875) (end 83.2125 42.9875) (width 0.25) (layer "B.Cu") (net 15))
 (segment (start 96.4 42.955723) (end 94.3 42.955723) (width 0.25) (layer "B.Cu") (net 15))
 (segment (start 100.4625 42.155723) (end 97.2 42.155723) (width 0.25) (layer "B.Cu") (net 15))
 (segment (start 83.2125 42.9875) (end 82.6 43.6) (width 0.25) (layer "B.Cu") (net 15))
 (segment (start 82.6 43.6) (end 81.3875 43.6) (width 0.25) (layer "B.Cu") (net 15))
 (segment (start 90.2 42.9875) (end 88.2 42.9875) (width 0.25) (layer "B.Cu") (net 15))
 (segment (start 88.2 42.9875) (end 85.3875 42.9875) (width 0.25) (layer "B.Cu") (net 15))
 (segment (start 97.2 42.155723) (end 96.4 42.955723) (width 0.25) (layer "B.Cu") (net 15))
 (segment (start 103.2625 48.25) (end 100.6625 48.25) (width 0.25) (layer "B.Cu") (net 15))
 (segment (start 92.2 42.9875) (end 90.2 42.9875) (width 0.25) (layer "B.Cu") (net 15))
 (segment (start 92.231777 42.955723) (end 92.2 42.9875) (width 0.25) (layer "B.Cu") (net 15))
 (segment (start 94.3 42.955723) (end 92.231777 42.955723) (width 0.25) (layer "B.Cu") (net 15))
 (segment (start 100.6625 48.25) (end 88.75 48.25) (width 0.25) (layer "B.Cu") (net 15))
 (segment (start 85.4 45.3) (end 85.4 43) (width 0.25) (layer "B.Cu") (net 15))
 (segment (start 109 42.15) (end 109 47.9) (width 0.25) (layer "B.Cu") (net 21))
 (segment (start 109 47.9) (end 104.3 47.9) (width 0.25) (layer "B.Cu") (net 21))
 (segment (start 104.3 47.9) (end 103.7 47.3) (width 0.25) (layer "B.Cu") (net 21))
 (segment (start 103.7 47.3) (end 102.5375 47.3) (width 0.25) (layer "B.Cu") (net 21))
 (segment (start 100.6625 46.35) (end 91.7375 46.35) (width 0.25) (layer "B.Cu") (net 16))
 (segment (start 91.7375 46.35) (end 90.2 44.8125) (width 0.25) (layer "B.Cu") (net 16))
 (segment (start 92.2 44.8125) (end 93.0875 45.7) (width 0.25) (layer "B.Cu") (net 19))
 (segment (start 102.6125 45.7) (end 103.2625 46.35) (width 0.25) (layer "B.Cu") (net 19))
 (segment (start 93.0875 45.7) (end 102.6125 45.7) (width 0.25) (layer "B.Cu") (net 19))
 (segment (start 76.7125 43.2) (end 76.6125 43.1) (width 0.25) (layer "B.Cu") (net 20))
 (segment (start 78.6125 43.2) (end 76.7125 43.2) (width 0.25) (layer "B.Cu") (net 20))
 (segment (start 52.5 40.5) (end 45.5 40.5) (width 0.25) (layer "B.Cu") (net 1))
 (segment (start 77.8 42.8) (end 77.1 42.1) (width 0.25) (layer "B.Cu") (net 1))
 (segment (start 59.9 40.9) (end 52.9 40.9) (width 0.25) (layer "B.Cu") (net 1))
 (segment (start 67.7 41.7) (end 67.3 41.3) (width 0.25) (layer "B.Cu") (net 1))
 (segment (start 78.6125 42.8) (end 77.8 42.8) (width 0.25) (layer "B.Cu") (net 1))
 (segment (start 77.1 42.1) (end 75.1 42.1) (width 0.25) (layer "B.Cu") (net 1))
 (segment (start 45.5 40.5) (end 44.8 39.8) (width 0.25) (layer "B.Cu") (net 1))
 (segment (start 74.7 41.7) (end 67.7 41.7) (width 0.25) (layer "B.Cu") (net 1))
 (segment (start 67.3 41.3) (end 60.3 41.3) (width 0.25) (layer "B.Cu") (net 1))
 (segment (start 52.9 40.9) (end 52.5 40.5) (width 0.25) (layer "B.Cu") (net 1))
 (segment (start 60.3 41.3) (end 59.9 40.9) (width 0.25) (layer "B.Cu") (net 1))
 (segment (start 44.8 39.8) (end 38.2 39.8) (width 0.25) (layer "B.Cu") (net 1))
 (segment (start 75.1 42.1) (end 74.7 41.7) (width 0.25) (layer "B.Cu") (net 1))
 (segment (start 53.1 40.5) (end 52.4 39.8) (width 0.25) (layer "B.Cu") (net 11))
 (segment (start 67.9 41.3) (end 67.5 40.9) (width 0.25) (layer "B.Cu") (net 11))
 (segment (start 52.4 39.8) (end 45.8 39.8) (width 0.25) (layer "B.Cu") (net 11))
 (segment (start 77.3 41.7) (end 75.3 41.7) (width 0.25) (layer "B.Cu") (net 11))
 (segment (start 78 42.4) (end 77.3 41.7) (width 0.25) (layer "B.Cu") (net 11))
 (segment (start 67.5 40.9) (end 60.5 40.9) (width 0.25) (layer "B.Cu") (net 11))
 (segment (start 74.9 41.3) (end 67.9 41.3) (width 0.25) (layer "B.Cu") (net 11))
 (segment (start 60.1 40.5) (end 53.1 40.5) (width 0.25) (layer "B.Cu") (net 11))
 (segment (start 60.5 40.9) (end 60.1 40.5) (width 0.25) (layer "B.Cu") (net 11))
 (segment (start 75.3 41.7) (end 74.9 41.3) (width 0.25) (layer "B.Cu") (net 11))
 (segment (start 78.6125 42.4) (end 78 42.4) (width 0.25) (layer "B.Cu") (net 11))
 (segment (start 75.1 40.9) (end 68.1 40.9) (width 0.25) (layer "B.Cu") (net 9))
 (segment (start 78.2 42) (end 77.5 41.3) (width 0.25) (layer "B.Cu") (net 9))
 (segment (start 75.5 41.3) (end 75.1 40.9) (width 0.25) (layer "B.Cu") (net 9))
 (segment (start 60.7 40.5) (end 60 39.8) (width 0.25) (layer "B.Cu") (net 9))
 (segment (start 67.7 40.5) (end 60.7 40.5) (width 0.25) (layer "B.Cu") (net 9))
 (segment (start 60 39.8) (end 53.4 39.8) (width 0.25) (layer "B.Cu") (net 9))
 (segment (start 68.1 40.9) (end 67.7 40.5) (width 0.25) (layer "B.Cu") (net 9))
 (segment (start 78.6125 42) (end 78.2 42) (width 0.25) (layer "B.Cu") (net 9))
 (segment (start 77.5 41.3) (end 75.5 41.3) (width 0.25) (layer "B.Cu") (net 9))
 (segment (start 75.7 40.9) (end 75.3 40.5) (width 0.25) (layer "B.Cu") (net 2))
 (segment (start 68.3 40.5) (end 67.6 39.8) (width 0.25) (layer "B.Cu") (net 2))
 (segment (start 79.2 40.9) (end 75.7 40.9) (width 0.25) (layer "B.Cu") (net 2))
 (segment (start 67.6 39.8) (end 61 39.8) (width 0.25) (layer "B.Cu") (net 2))
 (segment (start 75.3 40.5) (end 68.3 40.5) (width 0.25) (layer "B.Cu") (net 2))
 (segment (start 79.2 41.4125) (end 79.2 40.9) (width 0.25) (layer "B.Cu") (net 2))
 (segment (start 79.2 40.5) (end 75.9 40.5) (width 0.25) (layer "B.Cu") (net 5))
 (segment (start 75.9 40.5) (end 75.2 39.8) (width 0.25) (layer "B.Cu") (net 5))
 (segment (start 75.2 39.8) (end 68.6 39.8) (width 0.25) (layer "B.Cu") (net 5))
 (segment (start 79.6 41.4125) (end 79.6 40.9) (width 0.25) (layer "B.Cu") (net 5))
 (arc (start 79.6 40.9) (mid 79.482843 40.617157) (end 79.2 40.5) (width 0.25) (layer "B.Cu") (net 5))
 (segment (start 76.2 39.8) (end 79 39.8) (width 0.25) (layer "B.Cu") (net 6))
 (segment (start 80 40.8) (end 80 41.4125) (width 0.25) (layer "B.Cu") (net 6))
 (arc (start 79 39.8) (mid 79.707107 40.092893) (end 80 40.8) (width 0.25) (layer "B.Cu") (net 6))
 (segment (start 80.4 40.8) (end 80.4 41.4125) (width 0.25) (layer "B.Cu") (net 4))
 (segment (start 83.8 39.8) (end 81.4 39.8) (width 0.25) (layer "B.Cu") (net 4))
 (arc (start 80.4 40.8) (mid 80.692893 40.092893) (end 81.4 39.8) (width 0.25) (layer "B.Cu") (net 4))
 (segment (start 84.8 39.8) (end 91.4 39.8) (width 0.25) (layer "B.Cu") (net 8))
 (segment (start 81.2 40.5) (end 84.1 40.5) (width 0.25) (layer "B.Cu") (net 8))
 (segment (start 80.8 41.4125) (end 80.8 40.9) (width 0.25) (layer "B.Cu") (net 8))
 (segment (start 84.1 40.5) (end 84.8 39.8) (width 0.25) (layer "B.Cu") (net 8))
 (arc (start 80.8 40.9) (mid 80.917157 40.617157) (end 81.2 40.5) (width 0.25) (layer "B.Cu") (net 8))
 (segment (start 84.297705 40.902295) (end 82.897705 40.902295) (width 0.25) (layer "B.Cu") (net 7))
 (segment (start 81.8 42) (end 81.3875 42) (width 0.25) (layer "B.Cu") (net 7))
 (segment (start 92.4 39.8) (end 91.7 40.5) (width 0.25) (layer "B.Cu") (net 7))
 (segment (start 82.897705 40.902295) (end 81.8 42) (width 0.25) (layer "B.Cu") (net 7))
 (segment (start 99 39.8) (end 92.4 39.8) (width 0.25) (layer "B.Cu") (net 7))
 (segment (start 91.7 40.5) (end 84.7 40.5) (width 0.25) (layer "B.Cu") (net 7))
 (segment (start 84.7 40.5) (end 84.297705 40.902295) (width 0.25) (layer "B.Cu") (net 7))
 (segment (start 83.09837 41.30163) (end 84.49837 41.30163) (width 0.25) (layer "B.Cu") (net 12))
 (segment (start 99.3 40.5) (end 100 39.8) (width 0.25) (layer "B.Cu") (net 12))
 (segment (start 92.3 40.5) (end 99.3 40.5) (width 0.25) (layer "B.Cu") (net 12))
 (segment (start 84.49837 41.30163) (end 84.9 40.9) (width 0.25) (layer "B.Cu") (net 12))
 (segment (start 100 39.8) (end 106.6 39.8) (width 0.25) (layer "B.Cu") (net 12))
 (segment (start 91.9 40.9) (end 92.3 40.5) (width 0.25) (layer "B.Cu") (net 12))
 (segment (start 81.3875 42.4) (end 82 42.4) (width 0.25) (layer "B.Cu") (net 12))
 (segment (start 84.9 40.9) (end 91.9 40.9) (width 0.25) (layer "B.Cu") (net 12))
 (segment (start 82 42.4) (end 83.09837 41.30163) (width 0.25) (layer "B.Cu") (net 12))
 (segment (start 107.6 39.8) (end 114.2 39.8) (width 0.25) (layer "B.Cu") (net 3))
 (segment (start 85.1 41.3) (end 92.1 41.3) (width 0.25) (layer "B.Cu") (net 3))
 (segment (start 99.5 40.9) (end 99.9 40.5) (width 0.25) (layer "B.Cu") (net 3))
 (segment (start 92.1 41.3) (end 92.5 40.9) (width 0.25) (layer "B.Cu") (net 3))
 (segment (start 81.3875 42.8) (end 82.2 42.8) (width 0.25) (layer "B.Cu") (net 3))
 (segment (start 99.9 40.5) (end 106.9 40.5) (width 0.25) (layer "B.Cu") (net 3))
 (segment (start 106.9 40.5) (end 107.6 39.8) (width 0.25) (layer "B.Cu") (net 3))
 (segment (start 83.3 41.7) (end 84.696784 41.7) (width 0.25) (layer "B.Cu") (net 3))
 (segment (start 84.698392 41.701608) (end 85.1 41.3) (width 0.25) (layer "B.Cu") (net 3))
 (segment (start 82.2 42.8) (end 83.3 41.7) (width 0.25) (layer "B.Cu") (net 3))
 (segment (start 92.5 40.9) (end 99.5 40.9) (width 0.25) (layer "B.Cu") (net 3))
 (segment (start 84.696784 41.7) (end 84.698392 41.701608) (width 0.25) (layer "B.Cu") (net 3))
 (segment (start 114.55 40.5) (end 107.475432 40.5) (width 0.25) (layer "B.Cu") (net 10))
 (segment (start 99.71048 41.28952) (end 92.71048 41.28952) (width 0.25) (layer "B.Cu") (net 10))
 (segment (start 115.25 39.8) (end 114.55 40.5) (width 0.25) (layer "B.Cu") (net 10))
 (segment (start 121.8 39.8) (end 115.25 39.8) (width 0.25) (layer "B.Cu") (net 10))
 (segment (start 100.11048 40.88952) (end 99.71048 41.28952) (width 0.25) (layer "B.Cu") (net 10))
 (segment (start 92.71048 41.28952) (end 92.310481 41.689519) (width 0.25) (layer "B.Cu") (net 10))
 (segment (start 84.9 42.1) (end 83.5 42.1) (width 0.25) (layer "B.Cu") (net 10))
 (segment (start 92.310481 41.689519) (end 85.310481 41.689519) (width 0.25) (layer "B.Cu") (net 10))
 (segment (start 85.310481 41.689519) (end 84.9 42.1) (width 0.25) (layer "B.Cu") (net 10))
 (segment (start 83.5 42.1) (end 82.4 43.2) (width 0.25) (layer "B.Cu") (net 10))
 (segment (start 82.4 43.2) (end 81.3875 43.2) (width 0.25) (layer "B.Cu") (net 10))
 (segment (start 107.475432 40.5) (end 107.085912 40.88952) (width 0.25) (layer "B.Cu") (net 10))
 (segment (start 107.085912 40.88952) (end 100.11048 40.88952) (width 0.25) (layer "B.Cu") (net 10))
 (segment (start 108.2 47.3) (end 108.2 42.15) (width 0.25) (layer "B.Cu") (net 25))
 (segment (start 105.1375 47.3) (end 108.2 47.3) (width 0.25) (layer "B.Cu") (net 25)))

